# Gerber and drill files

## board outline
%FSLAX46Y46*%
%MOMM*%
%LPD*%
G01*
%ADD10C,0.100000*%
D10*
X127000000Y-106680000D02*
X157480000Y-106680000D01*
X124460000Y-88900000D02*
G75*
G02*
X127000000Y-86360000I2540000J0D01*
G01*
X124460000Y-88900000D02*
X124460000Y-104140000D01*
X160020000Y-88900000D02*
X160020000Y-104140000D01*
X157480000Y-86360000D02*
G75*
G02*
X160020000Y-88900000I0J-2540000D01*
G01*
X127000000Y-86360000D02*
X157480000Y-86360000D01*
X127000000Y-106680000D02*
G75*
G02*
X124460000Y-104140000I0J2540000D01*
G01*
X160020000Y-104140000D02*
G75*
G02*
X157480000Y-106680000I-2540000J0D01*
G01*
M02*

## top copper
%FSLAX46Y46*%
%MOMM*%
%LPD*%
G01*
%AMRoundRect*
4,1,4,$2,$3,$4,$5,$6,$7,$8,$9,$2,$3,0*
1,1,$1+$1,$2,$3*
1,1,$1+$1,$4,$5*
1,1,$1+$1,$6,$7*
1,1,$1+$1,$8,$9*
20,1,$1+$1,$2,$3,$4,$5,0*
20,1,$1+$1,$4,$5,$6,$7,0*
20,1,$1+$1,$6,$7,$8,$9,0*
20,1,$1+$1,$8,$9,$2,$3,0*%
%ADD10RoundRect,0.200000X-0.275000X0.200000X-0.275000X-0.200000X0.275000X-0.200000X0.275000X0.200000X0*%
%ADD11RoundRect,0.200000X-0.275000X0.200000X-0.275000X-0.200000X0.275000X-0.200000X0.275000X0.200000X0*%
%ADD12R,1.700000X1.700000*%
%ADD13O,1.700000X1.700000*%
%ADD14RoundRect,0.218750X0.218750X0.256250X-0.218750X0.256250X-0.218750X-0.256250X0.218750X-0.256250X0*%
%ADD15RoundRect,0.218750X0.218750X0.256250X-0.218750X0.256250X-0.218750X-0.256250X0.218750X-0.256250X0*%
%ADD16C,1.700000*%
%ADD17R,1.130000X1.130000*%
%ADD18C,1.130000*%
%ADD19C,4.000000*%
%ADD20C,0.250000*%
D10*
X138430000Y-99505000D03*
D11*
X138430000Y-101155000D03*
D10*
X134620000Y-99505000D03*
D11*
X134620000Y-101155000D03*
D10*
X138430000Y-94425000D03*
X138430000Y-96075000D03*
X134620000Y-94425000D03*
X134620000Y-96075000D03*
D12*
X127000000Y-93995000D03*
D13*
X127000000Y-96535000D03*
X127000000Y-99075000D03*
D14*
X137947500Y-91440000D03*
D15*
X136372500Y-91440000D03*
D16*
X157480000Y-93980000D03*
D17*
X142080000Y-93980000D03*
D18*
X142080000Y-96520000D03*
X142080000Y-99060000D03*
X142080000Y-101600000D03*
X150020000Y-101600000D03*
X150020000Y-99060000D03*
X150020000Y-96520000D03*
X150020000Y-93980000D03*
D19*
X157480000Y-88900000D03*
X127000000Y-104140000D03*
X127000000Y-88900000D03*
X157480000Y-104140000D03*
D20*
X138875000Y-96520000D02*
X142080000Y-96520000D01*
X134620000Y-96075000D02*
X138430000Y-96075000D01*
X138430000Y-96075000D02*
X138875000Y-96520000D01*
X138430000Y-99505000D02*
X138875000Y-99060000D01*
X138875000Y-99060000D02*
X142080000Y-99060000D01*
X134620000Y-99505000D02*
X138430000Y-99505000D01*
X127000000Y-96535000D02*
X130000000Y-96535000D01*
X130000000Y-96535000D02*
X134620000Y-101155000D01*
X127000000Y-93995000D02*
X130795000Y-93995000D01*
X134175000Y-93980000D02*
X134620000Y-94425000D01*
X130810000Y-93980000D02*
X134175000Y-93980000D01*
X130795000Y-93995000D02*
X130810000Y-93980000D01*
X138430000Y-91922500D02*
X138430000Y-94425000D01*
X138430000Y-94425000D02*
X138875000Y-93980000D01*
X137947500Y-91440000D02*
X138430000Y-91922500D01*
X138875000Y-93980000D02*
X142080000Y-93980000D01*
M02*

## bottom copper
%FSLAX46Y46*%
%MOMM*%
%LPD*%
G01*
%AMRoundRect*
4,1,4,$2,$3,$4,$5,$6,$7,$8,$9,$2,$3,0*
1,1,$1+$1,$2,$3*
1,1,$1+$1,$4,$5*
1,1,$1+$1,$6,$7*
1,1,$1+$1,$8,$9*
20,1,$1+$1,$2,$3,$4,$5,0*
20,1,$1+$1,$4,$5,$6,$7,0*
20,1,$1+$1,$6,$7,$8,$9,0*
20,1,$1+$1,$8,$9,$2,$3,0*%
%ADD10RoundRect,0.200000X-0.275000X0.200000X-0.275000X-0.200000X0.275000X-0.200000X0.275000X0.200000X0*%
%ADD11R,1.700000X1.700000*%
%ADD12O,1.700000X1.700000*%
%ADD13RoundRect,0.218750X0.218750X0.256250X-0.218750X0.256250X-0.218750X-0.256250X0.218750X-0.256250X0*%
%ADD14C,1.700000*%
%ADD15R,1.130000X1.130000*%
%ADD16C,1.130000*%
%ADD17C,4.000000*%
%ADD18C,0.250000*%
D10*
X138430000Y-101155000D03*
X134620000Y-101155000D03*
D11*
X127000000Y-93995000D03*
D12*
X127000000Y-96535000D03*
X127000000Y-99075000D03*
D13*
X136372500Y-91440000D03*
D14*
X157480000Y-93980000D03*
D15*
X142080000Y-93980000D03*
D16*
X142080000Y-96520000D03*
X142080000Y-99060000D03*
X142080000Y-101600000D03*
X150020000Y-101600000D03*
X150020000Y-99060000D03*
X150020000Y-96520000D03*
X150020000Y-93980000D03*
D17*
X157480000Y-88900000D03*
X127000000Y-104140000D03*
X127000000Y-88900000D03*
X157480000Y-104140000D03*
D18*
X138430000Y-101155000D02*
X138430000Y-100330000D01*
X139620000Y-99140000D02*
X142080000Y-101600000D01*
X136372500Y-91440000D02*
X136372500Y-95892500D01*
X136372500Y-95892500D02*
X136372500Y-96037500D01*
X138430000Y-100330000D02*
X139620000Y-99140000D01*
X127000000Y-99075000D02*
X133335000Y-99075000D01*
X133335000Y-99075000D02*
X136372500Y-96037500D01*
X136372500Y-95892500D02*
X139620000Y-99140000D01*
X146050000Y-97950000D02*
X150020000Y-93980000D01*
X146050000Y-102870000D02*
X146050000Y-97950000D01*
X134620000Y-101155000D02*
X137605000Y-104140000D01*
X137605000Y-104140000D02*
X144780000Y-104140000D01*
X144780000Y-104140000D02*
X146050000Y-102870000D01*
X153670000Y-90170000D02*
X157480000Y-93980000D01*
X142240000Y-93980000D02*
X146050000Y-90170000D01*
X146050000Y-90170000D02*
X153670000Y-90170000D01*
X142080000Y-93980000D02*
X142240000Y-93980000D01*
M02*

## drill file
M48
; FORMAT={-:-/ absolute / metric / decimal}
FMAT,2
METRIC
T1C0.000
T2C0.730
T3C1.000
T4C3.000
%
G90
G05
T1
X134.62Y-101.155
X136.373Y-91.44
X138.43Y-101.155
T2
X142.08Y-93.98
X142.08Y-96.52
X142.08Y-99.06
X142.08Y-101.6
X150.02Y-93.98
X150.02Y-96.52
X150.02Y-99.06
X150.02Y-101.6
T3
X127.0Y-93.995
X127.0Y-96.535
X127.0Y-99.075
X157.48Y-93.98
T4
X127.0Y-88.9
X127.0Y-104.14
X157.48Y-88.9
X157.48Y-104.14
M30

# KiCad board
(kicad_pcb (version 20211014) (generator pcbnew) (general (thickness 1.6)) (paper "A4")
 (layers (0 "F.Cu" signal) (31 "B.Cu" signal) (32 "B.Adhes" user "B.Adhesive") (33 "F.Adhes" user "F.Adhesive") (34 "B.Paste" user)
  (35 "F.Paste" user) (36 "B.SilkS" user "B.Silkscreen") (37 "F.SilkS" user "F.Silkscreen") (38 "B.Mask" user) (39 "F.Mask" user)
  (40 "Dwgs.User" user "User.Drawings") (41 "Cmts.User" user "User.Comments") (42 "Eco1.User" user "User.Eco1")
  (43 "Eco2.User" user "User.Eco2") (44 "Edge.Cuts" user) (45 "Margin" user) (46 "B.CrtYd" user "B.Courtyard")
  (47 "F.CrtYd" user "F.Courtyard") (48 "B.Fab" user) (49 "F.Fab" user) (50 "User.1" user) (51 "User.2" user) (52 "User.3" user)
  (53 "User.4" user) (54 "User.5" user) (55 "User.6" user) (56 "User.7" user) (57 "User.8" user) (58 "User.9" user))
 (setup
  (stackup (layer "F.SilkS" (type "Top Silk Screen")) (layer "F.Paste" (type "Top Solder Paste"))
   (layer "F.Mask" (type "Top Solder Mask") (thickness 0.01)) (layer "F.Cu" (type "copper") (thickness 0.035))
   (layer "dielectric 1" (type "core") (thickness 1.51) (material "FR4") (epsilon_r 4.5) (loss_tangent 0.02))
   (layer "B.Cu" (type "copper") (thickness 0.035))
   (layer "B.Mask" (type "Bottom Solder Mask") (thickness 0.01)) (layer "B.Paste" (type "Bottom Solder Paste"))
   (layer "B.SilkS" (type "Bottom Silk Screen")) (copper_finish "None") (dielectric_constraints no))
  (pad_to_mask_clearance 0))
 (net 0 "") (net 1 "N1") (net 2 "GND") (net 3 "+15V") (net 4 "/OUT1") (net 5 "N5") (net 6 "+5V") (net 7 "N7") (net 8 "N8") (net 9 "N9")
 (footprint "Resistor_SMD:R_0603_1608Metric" (layer "F.Cu") (at 138.43 100.33 -90)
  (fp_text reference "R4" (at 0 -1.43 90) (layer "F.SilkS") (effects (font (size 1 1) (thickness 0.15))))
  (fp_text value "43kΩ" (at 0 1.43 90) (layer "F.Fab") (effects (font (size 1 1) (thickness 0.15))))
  (pad "1" smd roundrect (at -0.825 0 270) (size 0.8 0.95) (layers "F.Cu" "F.Paste" "F.Mask") (roundrect_rratio 0.25) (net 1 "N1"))
  (pad "2" thru_hole roundrect (at 0.825 0 270) (size 0.8 0.95) (layers *.Cu *.Mask "F.Paste") (roundrect_rratio 0.25) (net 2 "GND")))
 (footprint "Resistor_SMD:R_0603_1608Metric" (layer "F.Cu") (at 134.62 100.33 -90)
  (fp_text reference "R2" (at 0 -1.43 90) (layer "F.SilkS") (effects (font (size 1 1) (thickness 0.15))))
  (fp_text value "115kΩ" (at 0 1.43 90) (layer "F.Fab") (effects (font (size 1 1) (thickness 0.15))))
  (pad "1" smd roundrect (at -0.825 0 270) (size 0.8 0.95) (layers "F.Cu" "F.Paste" "F.Mask") (roundrect_rratio 0.25) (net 1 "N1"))
  (pad "2" thru_hole roundrect (at 0.825 0 270) (size 0.8 0.95) (layers *.Cu *.Mask "F.Paste") (remove_unused_layers) (keep_end_layers)
   (roundrect_rratio 0.25) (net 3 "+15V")))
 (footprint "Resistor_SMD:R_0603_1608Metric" (layer "F.Cu") (at 138.43 95.25 -90)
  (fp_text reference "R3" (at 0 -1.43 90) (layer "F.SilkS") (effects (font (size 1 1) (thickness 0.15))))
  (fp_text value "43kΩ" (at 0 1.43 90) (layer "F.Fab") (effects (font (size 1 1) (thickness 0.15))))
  (pad "1" smd roundrect (at -0.825 0 270) (size 0.8 0.95) (layers "F.Cu" "F.Paste" "F.Mask") (roundrect_rratio 0.25) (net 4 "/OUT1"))
  (pad "2" smd roundrect (at 0.825 0 270) (size 0.8 0.95) (layers "F.Cu" "F.Paste" "F.Mask") (roundrect_rratio 0.25) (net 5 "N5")))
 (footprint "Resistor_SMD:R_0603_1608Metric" (layer "F.Cu") (at 134.62 95.25 -90)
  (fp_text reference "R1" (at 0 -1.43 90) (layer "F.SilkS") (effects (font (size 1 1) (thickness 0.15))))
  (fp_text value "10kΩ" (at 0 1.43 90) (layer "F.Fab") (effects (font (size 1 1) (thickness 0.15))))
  (pad "1" smd roundrect (at -0.825 0 270) (size 0.8 0.95) (layers "F.Cu" "F.Paste" "F.Mask") (roundrect_rratio 0.25) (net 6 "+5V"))
  (pad "2" smd roundrect (at 0.825 0 270) (size 0.8 0.95) (layers "F.Cu" "F.Paste" "F.Mask") (roundrect_rratio 0.25) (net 5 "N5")))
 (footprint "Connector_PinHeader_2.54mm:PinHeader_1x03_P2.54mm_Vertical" (layer "F.Cu") (at 127 93.995)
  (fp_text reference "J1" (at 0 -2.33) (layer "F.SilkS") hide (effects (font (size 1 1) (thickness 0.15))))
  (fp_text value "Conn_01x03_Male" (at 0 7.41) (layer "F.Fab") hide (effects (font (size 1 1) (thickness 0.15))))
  (pad "1" thru_hole rect (at 0 0) (size 1.7 1.7) (drill 1) (layers F&B.Cu *.Mask) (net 6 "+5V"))
  (pad "2" thru_hole oval (at 0 2.54) (size 1.7 1.7) (drill 1) (layers F&B.Cu *.Mask) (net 3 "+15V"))
  (pad "3" thru_hole oval (at 0 5.08) (size 1.7 1.7) (drill 1) (layers F&B.Cu *.Mask) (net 2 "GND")))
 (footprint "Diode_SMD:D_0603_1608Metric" (layer "F.Cu") (at 137.16 91.44 180)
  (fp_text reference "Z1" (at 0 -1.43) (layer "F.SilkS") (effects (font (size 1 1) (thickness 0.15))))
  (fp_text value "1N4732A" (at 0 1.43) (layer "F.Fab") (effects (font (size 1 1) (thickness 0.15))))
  (pad "1" smd roundrect (at -0.7875 0 180) (size 0.875 0.95) (layers "F.Cu" "F.Paste" "F.Mask") (roundrect_rratio 0.25) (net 4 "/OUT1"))
  (pad "2" thru_hole roundrect (at 0.7875 0 180) (size 0.875 0.95) (layers *.Cu *.Mask "F.Paste") (remove_unused_layers) (keep_end_layers)
   (roundrect_rratio 0.25) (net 2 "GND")))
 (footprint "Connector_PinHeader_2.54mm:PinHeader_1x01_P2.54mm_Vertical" (layer "F.Cu") (at 157.48 93.98)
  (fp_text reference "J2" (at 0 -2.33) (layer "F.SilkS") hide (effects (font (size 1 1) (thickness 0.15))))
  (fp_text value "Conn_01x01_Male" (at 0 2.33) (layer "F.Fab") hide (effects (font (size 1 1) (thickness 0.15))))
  (pad "1" thru_hole circle (at 0 0) (size 1.7 1.7) (drill 1) (layers *.Cu *.Mask) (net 4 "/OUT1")))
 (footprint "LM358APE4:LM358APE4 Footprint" (layer "F.Cu") (at 146.05 97.79)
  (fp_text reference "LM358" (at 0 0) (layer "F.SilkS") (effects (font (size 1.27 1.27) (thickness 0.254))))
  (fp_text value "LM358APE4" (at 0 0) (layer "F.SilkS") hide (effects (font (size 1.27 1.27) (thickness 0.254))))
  (pad "1" thru_hole rect (at -3.97 -3.81) (size 1.13 1.13) (drill 0.73) (layers *.Cu *.Mask) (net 4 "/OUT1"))
  (pad "2" thru_hole circle (at -3.97 -1.27) (size 1.13 1.13) (drill 0.73) (layers *.Cu *.Mask) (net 5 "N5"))
  (pad "3" thru_hole circle (at -3.97 1.27) (size 1.13 1.13) (drill 0.73) (layers *.Cu *.Mask) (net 1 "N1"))
  (pad "4" thru_hole circle (at -3.97 3.81) (size 1.13 1.13) (drill 0.73) (layers *.Cu *.Mask) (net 2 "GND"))
  (pad "5" thru_hole circle (at 3.97 3.81) (size 1.13 1.13) (drill 0.73) (layers *.Cu *.Mask) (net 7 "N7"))
  (pad "6" thru_hole circle (at 3.97 1.27) (size 1.13 1.13) (drill 0.73) (layers *.Cu *.Mask) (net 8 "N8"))
  (pad "7" thru_hole circle (at 3.97 -1.27) (size 1.13 1.13) (drill 0.73) (layers *.Cu *.Mask) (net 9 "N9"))
  (pad "8" thru_hole circle (at 3.97 -3.81) (size 1.13 1.13) (drill 0.73) (layers *.Cu *.Mask) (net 3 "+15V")))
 (gr_line (start 127 106.68) (end 157.48 106.68) (layer "Edge.Cuts") (width 0.1))
 (gr_arc (start 124.46 88.9) (mid 125.203949 87.103949) (end 127 86.36) (layer "Edge.Cuts") (width 0.1))
 (gr_line (start 124.46 88.9) (end 124.46 104.14) (layer "Edge.Cuts") (width 0.1))
 (gr_line (start 160.02 88.9) (end 160.02 104.14) (layer "Edge.Cuts") (width 0.1))
 (gr_arc (start 157.48 86.36) (mid 159.276051 87.103949) (end 160.02 88.9) (layer "Edge.Cuts") (width 0.1))
 (gr_line (start 127 86.36) (end 157.48 86.36) (layer "Edge.Cuts") (width 0.1))
 (gr_arc (start 127 106.68) (mid 125.203949 105.936051) (end 124.46 104.14) (layer "Edge.Cuts") (width 0.1))
 (gr_arc (start 160.02 104.14) (mid 159.276051 105.936051) (end 157.48 106.68) (layer "Edge.Cuts") (width 0.1))
 (via (at 157.48 88.9) (size 4) (drill 3) (layers "F.Cu" "B.Cu") (free) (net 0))
 (via (at 127 104.14) (size 4) (drill 3) (layers "F.Cu" "B.Cu") (free) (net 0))
 (via (at 127 88.9) (size 4) (drill 3) (layers "F.Cu" "B.Cu") (free) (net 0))
 (via (at 157.48 104.14) (size 4) (drill 3) (layers "F.Cu" "B.Cu") (free) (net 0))
 (segment (start 138.875 96.52) (end 142.08 96.52) (width 0.25) (layer "F.Cu") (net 5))
 (segment (start 134.62 96.075) (end 138.43 96.075) (width 0.25) (layer "F.Cu") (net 5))
 (segment (start 138.43 96.075) (end 138.875 96.52) (width 0.25) (layer "F.Cu") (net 5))
 (segment (start 138.43 99.505) (end 138.875 99.06) (width 0.25) (layer "F.Cu") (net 1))
 (segment (start 138.875 99.06) (end 142.08 99.06) (width 0.25) (layer "F.Cu") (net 1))
 (segment (start 134.62 99.505) (end 138.43 99.505) (width 0.25) (layer "F.Cu") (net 1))
 (segment (start 138.43 101.155) (end 138.43 100.33) (width 0.25) (layer "B.Cu") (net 2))
 (segment (start 139.62 99.14) (end 142.08 101.6) (width 0.25) (layer "B.Cu") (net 2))
 (segment (start 136.3725 91.44) (end 136.3725 95.8925) (width 0.25) (layer "B.Cu") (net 2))
 (segment (start 136.3725 95.8925) (end 136.3725 96.0375) (width 0.25) (layer "B.Cu") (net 2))
 (segment (start 138.43 100.33) (end 139.62 99.14) (width 0.25) (layer "B.Cu") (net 2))
 (segment (start 127 99.075) (end 133.335 99.075) (width 0.25) (layer "B.Cu") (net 2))
 (segment (start 133.335 99.075) (end 136.3725 96.0375) (width 0.25) (layer "B.Cu") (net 2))
 (segment (start 136.3725 95.8925) (end 139.62 99.14) (width 0.25) (layer "B.Cu") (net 2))
 (segment (start 127 96.535) (end 130 96.535) (width 0.25) (layer "F.Cu") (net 3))
 (segment (start 130 96.535) (end 134.62 101.155) (width 0.25) (layer "F.Cu") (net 3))
 (segment (start 146.05 97.95) (end 150.02 93.98) (width 0.25) (layer "B.Cu") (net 3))
 (segment (start 146.05 102.87) (end 146.05 97.95) (width 0.25) (layer "B.Cu") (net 3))
 (segment (start 134.62 101.155) (end 137.605 104.14) (width 0.25) (layer "B.Cu") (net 3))
 (segment (start 137.605 104.14) (end 144.78 104.14) (width 0.25) (layer "B.Cu") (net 3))
 (segment (start 144.78 104.14) (end 146.05 102.87) (width 0.25) (layer "B.Cu") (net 3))
 (segment (start 127 93.995) (end 130.795 93.995) (width 0.25) (layer "F.Cu") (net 6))
 (segment (start 134.175 93.98) (end 134.62 94.425) (width 0.25) (layer "F.Cu") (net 6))
 (segment (start 130.81 93.98) (end 134.175 93.98) (width 0.25) (layer "F.Cu") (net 6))
 (segment (start 130.795 93.995) (end 130.81 93.98) (width 0.25) (layer "F.Cu") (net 6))
 (segment (start 138.43 91.9225) (end 138.43 94.425) (width 0.25) (layer "F.Cu") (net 4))
 (segment (start 138.43 94.425) (end 138.875 93.98) (width 0.25) (layer "F.Cu") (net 4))
 (segment (start 137.9475 91.44) (end 138.43 91.9225) (width 0.25) (layer "F.Cu") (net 4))
 (segment (start 138.875 93.98) (end 142.08 93.98) (width 0.25) (layer "F.Cu") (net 4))
 (segment (start 153.67 90.17) (end 157.48 93.98) (width 0.25) (layer "B.Cu") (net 4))
 (segment (start 142.24 93.98) (end 146.05 90.17) (width 0.25) (layer "B.Cu") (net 4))
 (segment (start 146.05 90.17) (end 153.67 90.17) (width 0.25) (layer "B.Cu") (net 4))
 (segment (start 142.08 93.98) (end 142.24 93.98) (width 0.25) (layer "B.Cu") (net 4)))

